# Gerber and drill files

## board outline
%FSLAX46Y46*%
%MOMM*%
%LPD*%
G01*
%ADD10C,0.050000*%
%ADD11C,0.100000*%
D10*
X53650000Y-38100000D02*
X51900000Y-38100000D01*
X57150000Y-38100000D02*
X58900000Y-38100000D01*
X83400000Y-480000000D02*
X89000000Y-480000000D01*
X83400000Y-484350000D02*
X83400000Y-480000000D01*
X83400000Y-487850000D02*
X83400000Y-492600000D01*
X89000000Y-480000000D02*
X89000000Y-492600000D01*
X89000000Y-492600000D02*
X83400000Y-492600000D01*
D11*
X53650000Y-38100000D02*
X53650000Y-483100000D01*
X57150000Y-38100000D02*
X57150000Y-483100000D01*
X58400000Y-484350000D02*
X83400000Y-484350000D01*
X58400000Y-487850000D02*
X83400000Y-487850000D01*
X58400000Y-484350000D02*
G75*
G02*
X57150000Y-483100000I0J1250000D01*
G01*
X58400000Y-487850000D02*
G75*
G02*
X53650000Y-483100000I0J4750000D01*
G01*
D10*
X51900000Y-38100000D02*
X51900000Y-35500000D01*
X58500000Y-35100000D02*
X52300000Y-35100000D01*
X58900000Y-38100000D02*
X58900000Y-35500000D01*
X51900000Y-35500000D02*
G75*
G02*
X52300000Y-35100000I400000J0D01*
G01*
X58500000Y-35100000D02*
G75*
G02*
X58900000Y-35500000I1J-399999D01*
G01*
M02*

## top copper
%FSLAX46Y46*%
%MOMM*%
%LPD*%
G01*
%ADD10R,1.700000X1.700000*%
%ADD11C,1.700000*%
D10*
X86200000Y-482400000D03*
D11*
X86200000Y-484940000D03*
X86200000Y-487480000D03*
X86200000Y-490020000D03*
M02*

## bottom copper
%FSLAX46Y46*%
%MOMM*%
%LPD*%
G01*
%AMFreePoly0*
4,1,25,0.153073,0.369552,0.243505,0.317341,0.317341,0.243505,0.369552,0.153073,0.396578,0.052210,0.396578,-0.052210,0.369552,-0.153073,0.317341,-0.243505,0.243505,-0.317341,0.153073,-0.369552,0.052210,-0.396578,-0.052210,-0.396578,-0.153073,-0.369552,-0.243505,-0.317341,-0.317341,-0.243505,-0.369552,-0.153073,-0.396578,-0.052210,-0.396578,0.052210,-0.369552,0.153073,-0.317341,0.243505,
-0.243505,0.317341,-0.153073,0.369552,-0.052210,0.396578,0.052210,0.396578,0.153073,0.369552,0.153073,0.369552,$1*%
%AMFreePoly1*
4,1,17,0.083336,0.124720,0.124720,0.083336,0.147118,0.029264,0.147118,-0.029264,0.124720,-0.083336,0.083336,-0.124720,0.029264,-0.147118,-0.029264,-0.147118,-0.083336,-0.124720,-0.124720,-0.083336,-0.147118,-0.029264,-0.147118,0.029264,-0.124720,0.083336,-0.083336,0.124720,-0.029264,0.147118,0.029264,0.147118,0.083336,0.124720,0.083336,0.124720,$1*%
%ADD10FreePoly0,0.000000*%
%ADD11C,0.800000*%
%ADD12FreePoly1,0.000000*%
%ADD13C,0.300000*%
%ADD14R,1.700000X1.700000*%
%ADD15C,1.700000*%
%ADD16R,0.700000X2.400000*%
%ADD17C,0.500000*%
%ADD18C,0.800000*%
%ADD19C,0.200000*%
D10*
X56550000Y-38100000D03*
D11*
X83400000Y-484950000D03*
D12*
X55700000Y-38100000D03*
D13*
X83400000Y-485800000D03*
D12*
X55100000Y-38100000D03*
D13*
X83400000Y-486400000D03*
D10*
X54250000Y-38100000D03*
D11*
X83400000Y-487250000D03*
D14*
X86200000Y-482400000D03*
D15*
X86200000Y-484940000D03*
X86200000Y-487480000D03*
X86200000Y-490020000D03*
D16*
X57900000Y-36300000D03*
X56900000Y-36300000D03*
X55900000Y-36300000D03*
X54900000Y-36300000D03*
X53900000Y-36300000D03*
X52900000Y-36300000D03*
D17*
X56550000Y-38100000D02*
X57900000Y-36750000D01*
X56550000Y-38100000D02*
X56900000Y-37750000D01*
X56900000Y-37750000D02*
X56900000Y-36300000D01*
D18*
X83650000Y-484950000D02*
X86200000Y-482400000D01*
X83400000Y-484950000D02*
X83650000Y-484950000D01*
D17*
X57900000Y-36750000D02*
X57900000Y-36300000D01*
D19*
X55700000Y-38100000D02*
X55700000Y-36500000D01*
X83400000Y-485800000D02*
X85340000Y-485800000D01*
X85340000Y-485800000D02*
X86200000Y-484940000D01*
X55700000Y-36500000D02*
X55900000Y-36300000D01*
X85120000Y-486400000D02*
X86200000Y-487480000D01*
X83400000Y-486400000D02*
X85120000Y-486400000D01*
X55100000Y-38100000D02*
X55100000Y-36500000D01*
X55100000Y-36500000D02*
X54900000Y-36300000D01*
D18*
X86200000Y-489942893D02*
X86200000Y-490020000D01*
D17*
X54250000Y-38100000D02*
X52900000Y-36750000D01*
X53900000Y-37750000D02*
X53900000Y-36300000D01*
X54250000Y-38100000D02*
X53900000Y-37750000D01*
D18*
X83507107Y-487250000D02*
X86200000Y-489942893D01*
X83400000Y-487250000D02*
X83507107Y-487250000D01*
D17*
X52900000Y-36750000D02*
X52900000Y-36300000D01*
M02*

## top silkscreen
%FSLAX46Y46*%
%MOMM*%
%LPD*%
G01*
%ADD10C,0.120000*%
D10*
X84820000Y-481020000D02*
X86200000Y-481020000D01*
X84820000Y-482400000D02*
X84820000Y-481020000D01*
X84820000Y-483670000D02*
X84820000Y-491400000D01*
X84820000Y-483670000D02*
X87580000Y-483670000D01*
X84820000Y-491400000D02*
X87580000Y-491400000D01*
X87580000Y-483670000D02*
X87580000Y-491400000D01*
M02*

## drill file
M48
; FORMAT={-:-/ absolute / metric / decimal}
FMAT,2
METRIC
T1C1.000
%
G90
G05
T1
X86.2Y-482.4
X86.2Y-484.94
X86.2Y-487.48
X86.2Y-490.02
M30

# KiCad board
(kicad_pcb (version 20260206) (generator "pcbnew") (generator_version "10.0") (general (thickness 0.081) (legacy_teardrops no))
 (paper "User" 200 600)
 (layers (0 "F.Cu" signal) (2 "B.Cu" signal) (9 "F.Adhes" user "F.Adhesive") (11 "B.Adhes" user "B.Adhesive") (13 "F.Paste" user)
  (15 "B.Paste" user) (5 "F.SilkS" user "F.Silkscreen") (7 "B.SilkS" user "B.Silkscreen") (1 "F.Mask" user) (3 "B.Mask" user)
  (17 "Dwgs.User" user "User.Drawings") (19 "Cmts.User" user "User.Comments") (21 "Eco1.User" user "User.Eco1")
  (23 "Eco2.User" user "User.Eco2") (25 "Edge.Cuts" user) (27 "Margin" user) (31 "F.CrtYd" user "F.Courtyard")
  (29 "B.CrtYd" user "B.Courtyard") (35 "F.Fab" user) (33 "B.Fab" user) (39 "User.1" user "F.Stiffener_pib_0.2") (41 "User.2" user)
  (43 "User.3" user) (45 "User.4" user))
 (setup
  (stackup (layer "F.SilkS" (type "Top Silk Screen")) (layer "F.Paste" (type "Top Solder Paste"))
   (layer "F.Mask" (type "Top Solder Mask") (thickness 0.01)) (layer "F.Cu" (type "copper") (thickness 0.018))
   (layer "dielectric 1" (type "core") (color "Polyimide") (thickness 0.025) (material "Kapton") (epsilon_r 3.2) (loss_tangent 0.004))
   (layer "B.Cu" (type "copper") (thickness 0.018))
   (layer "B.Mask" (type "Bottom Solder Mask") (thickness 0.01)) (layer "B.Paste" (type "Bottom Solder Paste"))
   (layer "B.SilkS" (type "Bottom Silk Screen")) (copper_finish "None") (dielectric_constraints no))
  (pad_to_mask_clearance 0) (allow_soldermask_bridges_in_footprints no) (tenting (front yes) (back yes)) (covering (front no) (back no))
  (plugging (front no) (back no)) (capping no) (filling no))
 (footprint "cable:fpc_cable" (layer "F.Cu") (at 55.4 38.1)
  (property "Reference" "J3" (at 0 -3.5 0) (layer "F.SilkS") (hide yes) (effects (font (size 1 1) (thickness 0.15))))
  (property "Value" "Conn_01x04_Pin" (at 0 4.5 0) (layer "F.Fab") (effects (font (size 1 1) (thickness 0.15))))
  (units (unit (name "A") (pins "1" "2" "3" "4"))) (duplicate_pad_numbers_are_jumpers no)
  (fp_line (start -1.75 0) (end -1.75 445) (stroke (width 0.1) (type solid)) (layer "Edge.Cuts"))
  (fp_line (start 1.75 0) (end 1.75 445) (stroke (width 0.1) (type solid)) (layer "Edge.Cuts"))
  (fp_line (start 3 446.25) (end 28 446.25) (stroke (width 0.1) (type solid)) (layer "Edge.Cuts"))
  (fp_line (start 3 449.75) (end 28 449.75) (stroke (width 0.1) (type solid)) (layer "Edge.Cuts"))
  (fp_arc (start 3 446.25) (mid 2.116117 445.883883) (end 1.75 445) (stroke (width 0.1) (type solid)) (layer "Edge.Cuts"))
  (fp_arc (start 3 449.75) (mid -0.358757 448.358757) (end -1.75 445) (stroke (width 0.1) (type solid)) (layer "Edge.Cuts"))
  (pad "1" smd custom (at 1.15 0) (size 0.8 0.8) (layers "B.Cu") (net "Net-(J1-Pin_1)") (thermal_bridge_angle 90)
   (options (clearance outline) (anchor circle)) (primitives))
  (pad "1" smd circle (at 28 446.85) (size 0.8 0.8) (layers "B.Cu") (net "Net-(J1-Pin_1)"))
  (pad "2" smd custom (at 0.3 0) (size 0.3 0.3) (layers "B.Cu") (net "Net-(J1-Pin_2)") (thermal_bridge_angle 90)
   (options (clearance outline) (anchor circle)) (primitives))
  (pad "2" smd circle (at 28 447.7) (size 0.3 0.3) (layers "B.Cu") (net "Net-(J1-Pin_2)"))
  (pad "3" smd custom (at -0.3 0) (size 0.3 0.3) (layers "B.Cu") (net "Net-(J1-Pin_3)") (thermal_bridge_angle 90)
   (options (clearance outline) (anchor circle)) (primitives))
  (pad "3" smd circle (at 28 448.3) (size 0.3 0.3) (layers "B.Cu") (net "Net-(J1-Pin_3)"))
  (pad "4" smd custom (at -1.15 0) (size 0.8 0.8) (layers "B.Cu") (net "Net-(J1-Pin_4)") (thermal_bridge_angle 90)
   (options (clearance outline) (anchor circle)) (primitives))
  (pad "4" smd circle (at 28 449.15) (size 0.8 0.8) (layers "B.Cu") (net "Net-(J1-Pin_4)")))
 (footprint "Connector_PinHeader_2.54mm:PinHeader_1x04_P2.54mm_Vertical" (layer "F.Cu") (at 86.2 482.4)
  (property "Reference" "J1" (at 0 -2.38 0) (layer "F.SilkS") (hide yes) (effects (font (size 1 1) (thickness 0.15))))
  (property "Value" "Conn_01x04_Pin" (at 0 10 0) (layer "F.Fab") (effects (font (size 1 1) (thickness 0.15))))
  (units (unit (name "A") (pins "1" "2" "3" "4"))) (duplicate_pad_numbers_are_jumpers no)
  (fp_line (start -1.38 -1.38) (end 0 -1.38) (stroke (width 0.12) (type solid)) (layer "F.SilkS"))
  (fp_line (start -1.38 0) (end -1.38 -1.38) (stroke (width 0.12) (type solid)) (layer "F.SilkS"))
  (fp_line (start -1.38 1.27) (end -1.38 9) (stroke (width 0.12) (type solid)) (layer "F.SilkS"))
  (fp_line (start -1.38 1.27) (end 1.38 1.27) (stroke (width 0.12) (type solid)) (layer "F.SilkS"))
  (fp_line (start -1.38 9) (end 1.38 9) (stroke (width 0.12) (type solid)) (layer "F.SilkS"))
  (fp_line (start 1.38 1.27) (end 1.38 9) (stroke (width 0.12) (type solid)) (layer "F.SilkS"))
  (pad "1" thru_hole rect (at 0 0) (size 1.7 1.7) (drill 1) (layers "*.Cu" "*.Mask") (remove_unused_layers no) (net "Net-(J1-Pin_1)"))
  (pad "2" thru_hole circle (at 0 2.54) (size 1.7 1.7) (drill 1) (layers "*.Cu" "*.Mask") (remove_unused_layers no) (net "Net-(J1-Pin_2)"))
  (pad "3" thru_hole circle (at 0 5.08) (size 1.7 1.7) (drill 1) (layers "*.Cu" "*.Mask") (remove_unused_layers no) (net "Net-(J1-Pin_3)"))
  (pad "4" thru_hole circle (at 0 7.62) (size 1.7 1.7) (drill 1) (layers "*.Cu" "*.Mask") (remove_unused_layers no) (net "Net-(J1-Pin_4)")))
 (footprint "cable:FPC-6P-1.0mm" (layer "B.Cu") (at 57.9 36.3 180)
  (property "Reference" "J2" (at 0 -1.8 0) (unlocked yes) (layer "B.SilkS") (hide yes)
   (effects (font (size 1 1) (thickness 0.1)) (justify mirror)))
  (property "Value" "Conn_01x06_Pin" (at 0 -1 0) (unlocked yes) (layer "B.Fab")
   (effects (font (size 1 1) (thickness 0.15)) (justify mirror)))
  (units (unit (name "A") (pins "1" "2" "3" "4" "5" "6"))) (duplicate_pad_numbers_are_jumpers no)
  (fp_line (start 6 -1.8) (end 6 0.8) (stroke (width 0.05) (type default)) (layer "Edge.Cuts"))
  (fp_line (start -0.6 1.2) (end 5.6 1.2) (stroke (width 0.05) (type default)) (layer "Edge.Cuts"))
  (fp_line (start -1 -1.8) (end -1 0.8) (stroke (width 0.05) (type default)) (layer "Edge.Cuts"))
  (fp_arc (start 6 0.8) (mid 5.882843 1.082843) (end 5.6 1.2) (stroke (width 0.05) (type default)) (layer "Edge.Cuts"))
  (fp_arc (start -0.6 1.2) (mid -0.882843 1.082843) (end -1 0.8) (stroke (width 0.05) (type default)) (layer "Edge.Cuts"))
  (pad "1" smd rect (at 0 0 90) (size 2.4 0.7) (layers "B.Cu" "B.Mask" "B.Paste") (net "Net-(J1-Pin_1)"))
  (pad "2" smd rect (at 1 0 90) (size 2.4 0.7) (layers "B.Cu" "B.Mask" "B.Paste") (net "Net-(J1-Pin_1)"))
  (pad "3" smd rect (at 2 0 90) (size 2.4 0.7) (layers "B.Cu" "B.Mask" "B.Paste") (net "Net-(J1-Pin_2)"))
  (pad "4" smd rect (at 3 0 90) (size 2.4 0.7) (layers "B.Cu" "B.Mask" "B.Paste") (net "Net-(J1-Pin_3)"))
  (pad "5" smd rect (at 4 0 90) (size 2.4 0.7) (layers "B.Cu" "B.Mask" "B.Paste") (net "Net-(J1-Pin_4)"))
  (pad "6" smd rect (at 5 0 90) (size 2.4 0.7) (layers "B.Cu" "B.Mask" "B.Paste") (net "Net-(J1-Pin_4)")))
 (gr_line (start 53.65 38.1) (end 51.9 38.1) (stroke (width 0.05) (type default)) (layer "Edge.Cuts"))
 (gr_line (start 57.15 38.1) (end 58.9 38.1) (stroke (width 0.05) (type default)) (layer "Edge.Cuts"))
 (gr_line (start 83.4 480) (end 89 480) (stroke (width 0.05) (type default)) (layer "Edge.Cuts"))
 (gr_line (start 83.4 484.35) (end 83.4 480) (stroke (width 0.05) (type default)) (layer "Edge.Cuts"))
 (gr_line (start 83.4 487.85) (end 83.4 492.6) (stroke (width 0.05) (type solid)) (layer "Edge.Cuts"))
 (gr_line (start 89 480) (end 89 492.6) (stroke (width 0.05) (type default)) (layer "Edge.Cuts"))
 (gr_line (start 89 492.6) (end 83.4 492.6) (stroke (width 0.05) (type solid)) (layer "Edge.Cuts"))
 (segment (start 56.55 38.1) (end 57.9 36.75) (width 0.5) (layer "B.Cu") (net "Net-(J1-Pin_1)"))
 (segment (start 56.55 38.1) (end 56.9 37.75) (width 0.5) (layer "B.Cu") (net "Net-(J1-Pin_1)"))
 (segment (start 56.9 37.75) (end 56.9 36.3) (width 0.5) (layer "B.Cu") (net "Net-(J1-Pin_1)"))
 (segment (start 83.65 484.95) (end 86.2 482.4) (width 0.8) (layer "B.Cu") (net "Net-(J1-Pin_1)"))
 (segment (start 83.4 484.95) (end 83.65 484.95) (width 0.8) (layer "B.Cu") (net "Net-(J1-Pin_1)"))
 (segment (start 57.9 36.75) (end 57.9 36.3) (width 0.5) (layer "B.Cu") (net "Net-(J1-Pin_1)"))
 (segment (start 55.7 38.1) (end 55.7 36.5) (width 0.2) (layer "B.Cu") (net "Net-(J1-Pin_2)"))
 (segment (start 83.4 485.8) (end 85.34 485.8) (width 0.2) (layer "B.Cu") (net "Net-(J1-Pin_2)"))
 (segment (start 85.34 485.8) (end 86.2 484.94) (width 0.2) (layer "B.Cu") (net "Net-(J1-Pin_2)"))
 (segment (start 55.7 36.5) (end 55.9 36.3) (width 0.2) (layer "B.Cu") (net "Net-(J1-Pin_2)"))
 (segment (start 85.12 486.4) (end 86.2 487.48) (width 0.2) (layer "B.Cu") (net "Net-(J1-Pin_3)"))
 (segment (start 83.4 486.4) (end 85.12 486.4) (width 0.2) (layer "B.Cu") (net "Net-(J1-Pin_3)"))
 (segment (start 55.1 38.1) (end 55.1 36.5) (width 0.2) (layer "B.Cu") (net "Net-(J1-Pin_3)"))
 (segment (start 55.1 36.5) (end 54.9 36.3) (width 0.2) (layer "B.Cu") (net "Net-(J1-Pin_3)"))
 (segment (start 86.2 489.942893) (end 86.2 490.02) (width 0.8) (layer "B.Cu") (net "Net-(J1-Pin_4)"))
 (segment (start 54.25 38.1) (end 52.9 36.75) (width 0.5) (layer "B.Cu") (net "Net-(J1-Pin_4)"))
 (segment (start 53.9 37.75) (end 53.9 36.3) (width 0.5) (layer "B.Cu") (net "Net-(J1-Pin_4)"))
 (segment (start 54.25 38.1) (end 53.9 37.75) (width 0.5) (layer "B.Cu") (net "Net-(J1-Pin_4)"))
 (segment (start 83.507107 487.25) (end 86.2 489.942893) (width 0.8) (layer "B.Cu") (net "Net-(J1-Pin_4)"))
 (segment (start 83.4 487.25) (end 83.507107 487.25) (width 0.8) (layer "B.Cu") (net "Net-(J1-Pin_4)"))
 (segment (start 52.9 36.75) (end 52.9 36.3) (width 0.5) (layer "B.Cu") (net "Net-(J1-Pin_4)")))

